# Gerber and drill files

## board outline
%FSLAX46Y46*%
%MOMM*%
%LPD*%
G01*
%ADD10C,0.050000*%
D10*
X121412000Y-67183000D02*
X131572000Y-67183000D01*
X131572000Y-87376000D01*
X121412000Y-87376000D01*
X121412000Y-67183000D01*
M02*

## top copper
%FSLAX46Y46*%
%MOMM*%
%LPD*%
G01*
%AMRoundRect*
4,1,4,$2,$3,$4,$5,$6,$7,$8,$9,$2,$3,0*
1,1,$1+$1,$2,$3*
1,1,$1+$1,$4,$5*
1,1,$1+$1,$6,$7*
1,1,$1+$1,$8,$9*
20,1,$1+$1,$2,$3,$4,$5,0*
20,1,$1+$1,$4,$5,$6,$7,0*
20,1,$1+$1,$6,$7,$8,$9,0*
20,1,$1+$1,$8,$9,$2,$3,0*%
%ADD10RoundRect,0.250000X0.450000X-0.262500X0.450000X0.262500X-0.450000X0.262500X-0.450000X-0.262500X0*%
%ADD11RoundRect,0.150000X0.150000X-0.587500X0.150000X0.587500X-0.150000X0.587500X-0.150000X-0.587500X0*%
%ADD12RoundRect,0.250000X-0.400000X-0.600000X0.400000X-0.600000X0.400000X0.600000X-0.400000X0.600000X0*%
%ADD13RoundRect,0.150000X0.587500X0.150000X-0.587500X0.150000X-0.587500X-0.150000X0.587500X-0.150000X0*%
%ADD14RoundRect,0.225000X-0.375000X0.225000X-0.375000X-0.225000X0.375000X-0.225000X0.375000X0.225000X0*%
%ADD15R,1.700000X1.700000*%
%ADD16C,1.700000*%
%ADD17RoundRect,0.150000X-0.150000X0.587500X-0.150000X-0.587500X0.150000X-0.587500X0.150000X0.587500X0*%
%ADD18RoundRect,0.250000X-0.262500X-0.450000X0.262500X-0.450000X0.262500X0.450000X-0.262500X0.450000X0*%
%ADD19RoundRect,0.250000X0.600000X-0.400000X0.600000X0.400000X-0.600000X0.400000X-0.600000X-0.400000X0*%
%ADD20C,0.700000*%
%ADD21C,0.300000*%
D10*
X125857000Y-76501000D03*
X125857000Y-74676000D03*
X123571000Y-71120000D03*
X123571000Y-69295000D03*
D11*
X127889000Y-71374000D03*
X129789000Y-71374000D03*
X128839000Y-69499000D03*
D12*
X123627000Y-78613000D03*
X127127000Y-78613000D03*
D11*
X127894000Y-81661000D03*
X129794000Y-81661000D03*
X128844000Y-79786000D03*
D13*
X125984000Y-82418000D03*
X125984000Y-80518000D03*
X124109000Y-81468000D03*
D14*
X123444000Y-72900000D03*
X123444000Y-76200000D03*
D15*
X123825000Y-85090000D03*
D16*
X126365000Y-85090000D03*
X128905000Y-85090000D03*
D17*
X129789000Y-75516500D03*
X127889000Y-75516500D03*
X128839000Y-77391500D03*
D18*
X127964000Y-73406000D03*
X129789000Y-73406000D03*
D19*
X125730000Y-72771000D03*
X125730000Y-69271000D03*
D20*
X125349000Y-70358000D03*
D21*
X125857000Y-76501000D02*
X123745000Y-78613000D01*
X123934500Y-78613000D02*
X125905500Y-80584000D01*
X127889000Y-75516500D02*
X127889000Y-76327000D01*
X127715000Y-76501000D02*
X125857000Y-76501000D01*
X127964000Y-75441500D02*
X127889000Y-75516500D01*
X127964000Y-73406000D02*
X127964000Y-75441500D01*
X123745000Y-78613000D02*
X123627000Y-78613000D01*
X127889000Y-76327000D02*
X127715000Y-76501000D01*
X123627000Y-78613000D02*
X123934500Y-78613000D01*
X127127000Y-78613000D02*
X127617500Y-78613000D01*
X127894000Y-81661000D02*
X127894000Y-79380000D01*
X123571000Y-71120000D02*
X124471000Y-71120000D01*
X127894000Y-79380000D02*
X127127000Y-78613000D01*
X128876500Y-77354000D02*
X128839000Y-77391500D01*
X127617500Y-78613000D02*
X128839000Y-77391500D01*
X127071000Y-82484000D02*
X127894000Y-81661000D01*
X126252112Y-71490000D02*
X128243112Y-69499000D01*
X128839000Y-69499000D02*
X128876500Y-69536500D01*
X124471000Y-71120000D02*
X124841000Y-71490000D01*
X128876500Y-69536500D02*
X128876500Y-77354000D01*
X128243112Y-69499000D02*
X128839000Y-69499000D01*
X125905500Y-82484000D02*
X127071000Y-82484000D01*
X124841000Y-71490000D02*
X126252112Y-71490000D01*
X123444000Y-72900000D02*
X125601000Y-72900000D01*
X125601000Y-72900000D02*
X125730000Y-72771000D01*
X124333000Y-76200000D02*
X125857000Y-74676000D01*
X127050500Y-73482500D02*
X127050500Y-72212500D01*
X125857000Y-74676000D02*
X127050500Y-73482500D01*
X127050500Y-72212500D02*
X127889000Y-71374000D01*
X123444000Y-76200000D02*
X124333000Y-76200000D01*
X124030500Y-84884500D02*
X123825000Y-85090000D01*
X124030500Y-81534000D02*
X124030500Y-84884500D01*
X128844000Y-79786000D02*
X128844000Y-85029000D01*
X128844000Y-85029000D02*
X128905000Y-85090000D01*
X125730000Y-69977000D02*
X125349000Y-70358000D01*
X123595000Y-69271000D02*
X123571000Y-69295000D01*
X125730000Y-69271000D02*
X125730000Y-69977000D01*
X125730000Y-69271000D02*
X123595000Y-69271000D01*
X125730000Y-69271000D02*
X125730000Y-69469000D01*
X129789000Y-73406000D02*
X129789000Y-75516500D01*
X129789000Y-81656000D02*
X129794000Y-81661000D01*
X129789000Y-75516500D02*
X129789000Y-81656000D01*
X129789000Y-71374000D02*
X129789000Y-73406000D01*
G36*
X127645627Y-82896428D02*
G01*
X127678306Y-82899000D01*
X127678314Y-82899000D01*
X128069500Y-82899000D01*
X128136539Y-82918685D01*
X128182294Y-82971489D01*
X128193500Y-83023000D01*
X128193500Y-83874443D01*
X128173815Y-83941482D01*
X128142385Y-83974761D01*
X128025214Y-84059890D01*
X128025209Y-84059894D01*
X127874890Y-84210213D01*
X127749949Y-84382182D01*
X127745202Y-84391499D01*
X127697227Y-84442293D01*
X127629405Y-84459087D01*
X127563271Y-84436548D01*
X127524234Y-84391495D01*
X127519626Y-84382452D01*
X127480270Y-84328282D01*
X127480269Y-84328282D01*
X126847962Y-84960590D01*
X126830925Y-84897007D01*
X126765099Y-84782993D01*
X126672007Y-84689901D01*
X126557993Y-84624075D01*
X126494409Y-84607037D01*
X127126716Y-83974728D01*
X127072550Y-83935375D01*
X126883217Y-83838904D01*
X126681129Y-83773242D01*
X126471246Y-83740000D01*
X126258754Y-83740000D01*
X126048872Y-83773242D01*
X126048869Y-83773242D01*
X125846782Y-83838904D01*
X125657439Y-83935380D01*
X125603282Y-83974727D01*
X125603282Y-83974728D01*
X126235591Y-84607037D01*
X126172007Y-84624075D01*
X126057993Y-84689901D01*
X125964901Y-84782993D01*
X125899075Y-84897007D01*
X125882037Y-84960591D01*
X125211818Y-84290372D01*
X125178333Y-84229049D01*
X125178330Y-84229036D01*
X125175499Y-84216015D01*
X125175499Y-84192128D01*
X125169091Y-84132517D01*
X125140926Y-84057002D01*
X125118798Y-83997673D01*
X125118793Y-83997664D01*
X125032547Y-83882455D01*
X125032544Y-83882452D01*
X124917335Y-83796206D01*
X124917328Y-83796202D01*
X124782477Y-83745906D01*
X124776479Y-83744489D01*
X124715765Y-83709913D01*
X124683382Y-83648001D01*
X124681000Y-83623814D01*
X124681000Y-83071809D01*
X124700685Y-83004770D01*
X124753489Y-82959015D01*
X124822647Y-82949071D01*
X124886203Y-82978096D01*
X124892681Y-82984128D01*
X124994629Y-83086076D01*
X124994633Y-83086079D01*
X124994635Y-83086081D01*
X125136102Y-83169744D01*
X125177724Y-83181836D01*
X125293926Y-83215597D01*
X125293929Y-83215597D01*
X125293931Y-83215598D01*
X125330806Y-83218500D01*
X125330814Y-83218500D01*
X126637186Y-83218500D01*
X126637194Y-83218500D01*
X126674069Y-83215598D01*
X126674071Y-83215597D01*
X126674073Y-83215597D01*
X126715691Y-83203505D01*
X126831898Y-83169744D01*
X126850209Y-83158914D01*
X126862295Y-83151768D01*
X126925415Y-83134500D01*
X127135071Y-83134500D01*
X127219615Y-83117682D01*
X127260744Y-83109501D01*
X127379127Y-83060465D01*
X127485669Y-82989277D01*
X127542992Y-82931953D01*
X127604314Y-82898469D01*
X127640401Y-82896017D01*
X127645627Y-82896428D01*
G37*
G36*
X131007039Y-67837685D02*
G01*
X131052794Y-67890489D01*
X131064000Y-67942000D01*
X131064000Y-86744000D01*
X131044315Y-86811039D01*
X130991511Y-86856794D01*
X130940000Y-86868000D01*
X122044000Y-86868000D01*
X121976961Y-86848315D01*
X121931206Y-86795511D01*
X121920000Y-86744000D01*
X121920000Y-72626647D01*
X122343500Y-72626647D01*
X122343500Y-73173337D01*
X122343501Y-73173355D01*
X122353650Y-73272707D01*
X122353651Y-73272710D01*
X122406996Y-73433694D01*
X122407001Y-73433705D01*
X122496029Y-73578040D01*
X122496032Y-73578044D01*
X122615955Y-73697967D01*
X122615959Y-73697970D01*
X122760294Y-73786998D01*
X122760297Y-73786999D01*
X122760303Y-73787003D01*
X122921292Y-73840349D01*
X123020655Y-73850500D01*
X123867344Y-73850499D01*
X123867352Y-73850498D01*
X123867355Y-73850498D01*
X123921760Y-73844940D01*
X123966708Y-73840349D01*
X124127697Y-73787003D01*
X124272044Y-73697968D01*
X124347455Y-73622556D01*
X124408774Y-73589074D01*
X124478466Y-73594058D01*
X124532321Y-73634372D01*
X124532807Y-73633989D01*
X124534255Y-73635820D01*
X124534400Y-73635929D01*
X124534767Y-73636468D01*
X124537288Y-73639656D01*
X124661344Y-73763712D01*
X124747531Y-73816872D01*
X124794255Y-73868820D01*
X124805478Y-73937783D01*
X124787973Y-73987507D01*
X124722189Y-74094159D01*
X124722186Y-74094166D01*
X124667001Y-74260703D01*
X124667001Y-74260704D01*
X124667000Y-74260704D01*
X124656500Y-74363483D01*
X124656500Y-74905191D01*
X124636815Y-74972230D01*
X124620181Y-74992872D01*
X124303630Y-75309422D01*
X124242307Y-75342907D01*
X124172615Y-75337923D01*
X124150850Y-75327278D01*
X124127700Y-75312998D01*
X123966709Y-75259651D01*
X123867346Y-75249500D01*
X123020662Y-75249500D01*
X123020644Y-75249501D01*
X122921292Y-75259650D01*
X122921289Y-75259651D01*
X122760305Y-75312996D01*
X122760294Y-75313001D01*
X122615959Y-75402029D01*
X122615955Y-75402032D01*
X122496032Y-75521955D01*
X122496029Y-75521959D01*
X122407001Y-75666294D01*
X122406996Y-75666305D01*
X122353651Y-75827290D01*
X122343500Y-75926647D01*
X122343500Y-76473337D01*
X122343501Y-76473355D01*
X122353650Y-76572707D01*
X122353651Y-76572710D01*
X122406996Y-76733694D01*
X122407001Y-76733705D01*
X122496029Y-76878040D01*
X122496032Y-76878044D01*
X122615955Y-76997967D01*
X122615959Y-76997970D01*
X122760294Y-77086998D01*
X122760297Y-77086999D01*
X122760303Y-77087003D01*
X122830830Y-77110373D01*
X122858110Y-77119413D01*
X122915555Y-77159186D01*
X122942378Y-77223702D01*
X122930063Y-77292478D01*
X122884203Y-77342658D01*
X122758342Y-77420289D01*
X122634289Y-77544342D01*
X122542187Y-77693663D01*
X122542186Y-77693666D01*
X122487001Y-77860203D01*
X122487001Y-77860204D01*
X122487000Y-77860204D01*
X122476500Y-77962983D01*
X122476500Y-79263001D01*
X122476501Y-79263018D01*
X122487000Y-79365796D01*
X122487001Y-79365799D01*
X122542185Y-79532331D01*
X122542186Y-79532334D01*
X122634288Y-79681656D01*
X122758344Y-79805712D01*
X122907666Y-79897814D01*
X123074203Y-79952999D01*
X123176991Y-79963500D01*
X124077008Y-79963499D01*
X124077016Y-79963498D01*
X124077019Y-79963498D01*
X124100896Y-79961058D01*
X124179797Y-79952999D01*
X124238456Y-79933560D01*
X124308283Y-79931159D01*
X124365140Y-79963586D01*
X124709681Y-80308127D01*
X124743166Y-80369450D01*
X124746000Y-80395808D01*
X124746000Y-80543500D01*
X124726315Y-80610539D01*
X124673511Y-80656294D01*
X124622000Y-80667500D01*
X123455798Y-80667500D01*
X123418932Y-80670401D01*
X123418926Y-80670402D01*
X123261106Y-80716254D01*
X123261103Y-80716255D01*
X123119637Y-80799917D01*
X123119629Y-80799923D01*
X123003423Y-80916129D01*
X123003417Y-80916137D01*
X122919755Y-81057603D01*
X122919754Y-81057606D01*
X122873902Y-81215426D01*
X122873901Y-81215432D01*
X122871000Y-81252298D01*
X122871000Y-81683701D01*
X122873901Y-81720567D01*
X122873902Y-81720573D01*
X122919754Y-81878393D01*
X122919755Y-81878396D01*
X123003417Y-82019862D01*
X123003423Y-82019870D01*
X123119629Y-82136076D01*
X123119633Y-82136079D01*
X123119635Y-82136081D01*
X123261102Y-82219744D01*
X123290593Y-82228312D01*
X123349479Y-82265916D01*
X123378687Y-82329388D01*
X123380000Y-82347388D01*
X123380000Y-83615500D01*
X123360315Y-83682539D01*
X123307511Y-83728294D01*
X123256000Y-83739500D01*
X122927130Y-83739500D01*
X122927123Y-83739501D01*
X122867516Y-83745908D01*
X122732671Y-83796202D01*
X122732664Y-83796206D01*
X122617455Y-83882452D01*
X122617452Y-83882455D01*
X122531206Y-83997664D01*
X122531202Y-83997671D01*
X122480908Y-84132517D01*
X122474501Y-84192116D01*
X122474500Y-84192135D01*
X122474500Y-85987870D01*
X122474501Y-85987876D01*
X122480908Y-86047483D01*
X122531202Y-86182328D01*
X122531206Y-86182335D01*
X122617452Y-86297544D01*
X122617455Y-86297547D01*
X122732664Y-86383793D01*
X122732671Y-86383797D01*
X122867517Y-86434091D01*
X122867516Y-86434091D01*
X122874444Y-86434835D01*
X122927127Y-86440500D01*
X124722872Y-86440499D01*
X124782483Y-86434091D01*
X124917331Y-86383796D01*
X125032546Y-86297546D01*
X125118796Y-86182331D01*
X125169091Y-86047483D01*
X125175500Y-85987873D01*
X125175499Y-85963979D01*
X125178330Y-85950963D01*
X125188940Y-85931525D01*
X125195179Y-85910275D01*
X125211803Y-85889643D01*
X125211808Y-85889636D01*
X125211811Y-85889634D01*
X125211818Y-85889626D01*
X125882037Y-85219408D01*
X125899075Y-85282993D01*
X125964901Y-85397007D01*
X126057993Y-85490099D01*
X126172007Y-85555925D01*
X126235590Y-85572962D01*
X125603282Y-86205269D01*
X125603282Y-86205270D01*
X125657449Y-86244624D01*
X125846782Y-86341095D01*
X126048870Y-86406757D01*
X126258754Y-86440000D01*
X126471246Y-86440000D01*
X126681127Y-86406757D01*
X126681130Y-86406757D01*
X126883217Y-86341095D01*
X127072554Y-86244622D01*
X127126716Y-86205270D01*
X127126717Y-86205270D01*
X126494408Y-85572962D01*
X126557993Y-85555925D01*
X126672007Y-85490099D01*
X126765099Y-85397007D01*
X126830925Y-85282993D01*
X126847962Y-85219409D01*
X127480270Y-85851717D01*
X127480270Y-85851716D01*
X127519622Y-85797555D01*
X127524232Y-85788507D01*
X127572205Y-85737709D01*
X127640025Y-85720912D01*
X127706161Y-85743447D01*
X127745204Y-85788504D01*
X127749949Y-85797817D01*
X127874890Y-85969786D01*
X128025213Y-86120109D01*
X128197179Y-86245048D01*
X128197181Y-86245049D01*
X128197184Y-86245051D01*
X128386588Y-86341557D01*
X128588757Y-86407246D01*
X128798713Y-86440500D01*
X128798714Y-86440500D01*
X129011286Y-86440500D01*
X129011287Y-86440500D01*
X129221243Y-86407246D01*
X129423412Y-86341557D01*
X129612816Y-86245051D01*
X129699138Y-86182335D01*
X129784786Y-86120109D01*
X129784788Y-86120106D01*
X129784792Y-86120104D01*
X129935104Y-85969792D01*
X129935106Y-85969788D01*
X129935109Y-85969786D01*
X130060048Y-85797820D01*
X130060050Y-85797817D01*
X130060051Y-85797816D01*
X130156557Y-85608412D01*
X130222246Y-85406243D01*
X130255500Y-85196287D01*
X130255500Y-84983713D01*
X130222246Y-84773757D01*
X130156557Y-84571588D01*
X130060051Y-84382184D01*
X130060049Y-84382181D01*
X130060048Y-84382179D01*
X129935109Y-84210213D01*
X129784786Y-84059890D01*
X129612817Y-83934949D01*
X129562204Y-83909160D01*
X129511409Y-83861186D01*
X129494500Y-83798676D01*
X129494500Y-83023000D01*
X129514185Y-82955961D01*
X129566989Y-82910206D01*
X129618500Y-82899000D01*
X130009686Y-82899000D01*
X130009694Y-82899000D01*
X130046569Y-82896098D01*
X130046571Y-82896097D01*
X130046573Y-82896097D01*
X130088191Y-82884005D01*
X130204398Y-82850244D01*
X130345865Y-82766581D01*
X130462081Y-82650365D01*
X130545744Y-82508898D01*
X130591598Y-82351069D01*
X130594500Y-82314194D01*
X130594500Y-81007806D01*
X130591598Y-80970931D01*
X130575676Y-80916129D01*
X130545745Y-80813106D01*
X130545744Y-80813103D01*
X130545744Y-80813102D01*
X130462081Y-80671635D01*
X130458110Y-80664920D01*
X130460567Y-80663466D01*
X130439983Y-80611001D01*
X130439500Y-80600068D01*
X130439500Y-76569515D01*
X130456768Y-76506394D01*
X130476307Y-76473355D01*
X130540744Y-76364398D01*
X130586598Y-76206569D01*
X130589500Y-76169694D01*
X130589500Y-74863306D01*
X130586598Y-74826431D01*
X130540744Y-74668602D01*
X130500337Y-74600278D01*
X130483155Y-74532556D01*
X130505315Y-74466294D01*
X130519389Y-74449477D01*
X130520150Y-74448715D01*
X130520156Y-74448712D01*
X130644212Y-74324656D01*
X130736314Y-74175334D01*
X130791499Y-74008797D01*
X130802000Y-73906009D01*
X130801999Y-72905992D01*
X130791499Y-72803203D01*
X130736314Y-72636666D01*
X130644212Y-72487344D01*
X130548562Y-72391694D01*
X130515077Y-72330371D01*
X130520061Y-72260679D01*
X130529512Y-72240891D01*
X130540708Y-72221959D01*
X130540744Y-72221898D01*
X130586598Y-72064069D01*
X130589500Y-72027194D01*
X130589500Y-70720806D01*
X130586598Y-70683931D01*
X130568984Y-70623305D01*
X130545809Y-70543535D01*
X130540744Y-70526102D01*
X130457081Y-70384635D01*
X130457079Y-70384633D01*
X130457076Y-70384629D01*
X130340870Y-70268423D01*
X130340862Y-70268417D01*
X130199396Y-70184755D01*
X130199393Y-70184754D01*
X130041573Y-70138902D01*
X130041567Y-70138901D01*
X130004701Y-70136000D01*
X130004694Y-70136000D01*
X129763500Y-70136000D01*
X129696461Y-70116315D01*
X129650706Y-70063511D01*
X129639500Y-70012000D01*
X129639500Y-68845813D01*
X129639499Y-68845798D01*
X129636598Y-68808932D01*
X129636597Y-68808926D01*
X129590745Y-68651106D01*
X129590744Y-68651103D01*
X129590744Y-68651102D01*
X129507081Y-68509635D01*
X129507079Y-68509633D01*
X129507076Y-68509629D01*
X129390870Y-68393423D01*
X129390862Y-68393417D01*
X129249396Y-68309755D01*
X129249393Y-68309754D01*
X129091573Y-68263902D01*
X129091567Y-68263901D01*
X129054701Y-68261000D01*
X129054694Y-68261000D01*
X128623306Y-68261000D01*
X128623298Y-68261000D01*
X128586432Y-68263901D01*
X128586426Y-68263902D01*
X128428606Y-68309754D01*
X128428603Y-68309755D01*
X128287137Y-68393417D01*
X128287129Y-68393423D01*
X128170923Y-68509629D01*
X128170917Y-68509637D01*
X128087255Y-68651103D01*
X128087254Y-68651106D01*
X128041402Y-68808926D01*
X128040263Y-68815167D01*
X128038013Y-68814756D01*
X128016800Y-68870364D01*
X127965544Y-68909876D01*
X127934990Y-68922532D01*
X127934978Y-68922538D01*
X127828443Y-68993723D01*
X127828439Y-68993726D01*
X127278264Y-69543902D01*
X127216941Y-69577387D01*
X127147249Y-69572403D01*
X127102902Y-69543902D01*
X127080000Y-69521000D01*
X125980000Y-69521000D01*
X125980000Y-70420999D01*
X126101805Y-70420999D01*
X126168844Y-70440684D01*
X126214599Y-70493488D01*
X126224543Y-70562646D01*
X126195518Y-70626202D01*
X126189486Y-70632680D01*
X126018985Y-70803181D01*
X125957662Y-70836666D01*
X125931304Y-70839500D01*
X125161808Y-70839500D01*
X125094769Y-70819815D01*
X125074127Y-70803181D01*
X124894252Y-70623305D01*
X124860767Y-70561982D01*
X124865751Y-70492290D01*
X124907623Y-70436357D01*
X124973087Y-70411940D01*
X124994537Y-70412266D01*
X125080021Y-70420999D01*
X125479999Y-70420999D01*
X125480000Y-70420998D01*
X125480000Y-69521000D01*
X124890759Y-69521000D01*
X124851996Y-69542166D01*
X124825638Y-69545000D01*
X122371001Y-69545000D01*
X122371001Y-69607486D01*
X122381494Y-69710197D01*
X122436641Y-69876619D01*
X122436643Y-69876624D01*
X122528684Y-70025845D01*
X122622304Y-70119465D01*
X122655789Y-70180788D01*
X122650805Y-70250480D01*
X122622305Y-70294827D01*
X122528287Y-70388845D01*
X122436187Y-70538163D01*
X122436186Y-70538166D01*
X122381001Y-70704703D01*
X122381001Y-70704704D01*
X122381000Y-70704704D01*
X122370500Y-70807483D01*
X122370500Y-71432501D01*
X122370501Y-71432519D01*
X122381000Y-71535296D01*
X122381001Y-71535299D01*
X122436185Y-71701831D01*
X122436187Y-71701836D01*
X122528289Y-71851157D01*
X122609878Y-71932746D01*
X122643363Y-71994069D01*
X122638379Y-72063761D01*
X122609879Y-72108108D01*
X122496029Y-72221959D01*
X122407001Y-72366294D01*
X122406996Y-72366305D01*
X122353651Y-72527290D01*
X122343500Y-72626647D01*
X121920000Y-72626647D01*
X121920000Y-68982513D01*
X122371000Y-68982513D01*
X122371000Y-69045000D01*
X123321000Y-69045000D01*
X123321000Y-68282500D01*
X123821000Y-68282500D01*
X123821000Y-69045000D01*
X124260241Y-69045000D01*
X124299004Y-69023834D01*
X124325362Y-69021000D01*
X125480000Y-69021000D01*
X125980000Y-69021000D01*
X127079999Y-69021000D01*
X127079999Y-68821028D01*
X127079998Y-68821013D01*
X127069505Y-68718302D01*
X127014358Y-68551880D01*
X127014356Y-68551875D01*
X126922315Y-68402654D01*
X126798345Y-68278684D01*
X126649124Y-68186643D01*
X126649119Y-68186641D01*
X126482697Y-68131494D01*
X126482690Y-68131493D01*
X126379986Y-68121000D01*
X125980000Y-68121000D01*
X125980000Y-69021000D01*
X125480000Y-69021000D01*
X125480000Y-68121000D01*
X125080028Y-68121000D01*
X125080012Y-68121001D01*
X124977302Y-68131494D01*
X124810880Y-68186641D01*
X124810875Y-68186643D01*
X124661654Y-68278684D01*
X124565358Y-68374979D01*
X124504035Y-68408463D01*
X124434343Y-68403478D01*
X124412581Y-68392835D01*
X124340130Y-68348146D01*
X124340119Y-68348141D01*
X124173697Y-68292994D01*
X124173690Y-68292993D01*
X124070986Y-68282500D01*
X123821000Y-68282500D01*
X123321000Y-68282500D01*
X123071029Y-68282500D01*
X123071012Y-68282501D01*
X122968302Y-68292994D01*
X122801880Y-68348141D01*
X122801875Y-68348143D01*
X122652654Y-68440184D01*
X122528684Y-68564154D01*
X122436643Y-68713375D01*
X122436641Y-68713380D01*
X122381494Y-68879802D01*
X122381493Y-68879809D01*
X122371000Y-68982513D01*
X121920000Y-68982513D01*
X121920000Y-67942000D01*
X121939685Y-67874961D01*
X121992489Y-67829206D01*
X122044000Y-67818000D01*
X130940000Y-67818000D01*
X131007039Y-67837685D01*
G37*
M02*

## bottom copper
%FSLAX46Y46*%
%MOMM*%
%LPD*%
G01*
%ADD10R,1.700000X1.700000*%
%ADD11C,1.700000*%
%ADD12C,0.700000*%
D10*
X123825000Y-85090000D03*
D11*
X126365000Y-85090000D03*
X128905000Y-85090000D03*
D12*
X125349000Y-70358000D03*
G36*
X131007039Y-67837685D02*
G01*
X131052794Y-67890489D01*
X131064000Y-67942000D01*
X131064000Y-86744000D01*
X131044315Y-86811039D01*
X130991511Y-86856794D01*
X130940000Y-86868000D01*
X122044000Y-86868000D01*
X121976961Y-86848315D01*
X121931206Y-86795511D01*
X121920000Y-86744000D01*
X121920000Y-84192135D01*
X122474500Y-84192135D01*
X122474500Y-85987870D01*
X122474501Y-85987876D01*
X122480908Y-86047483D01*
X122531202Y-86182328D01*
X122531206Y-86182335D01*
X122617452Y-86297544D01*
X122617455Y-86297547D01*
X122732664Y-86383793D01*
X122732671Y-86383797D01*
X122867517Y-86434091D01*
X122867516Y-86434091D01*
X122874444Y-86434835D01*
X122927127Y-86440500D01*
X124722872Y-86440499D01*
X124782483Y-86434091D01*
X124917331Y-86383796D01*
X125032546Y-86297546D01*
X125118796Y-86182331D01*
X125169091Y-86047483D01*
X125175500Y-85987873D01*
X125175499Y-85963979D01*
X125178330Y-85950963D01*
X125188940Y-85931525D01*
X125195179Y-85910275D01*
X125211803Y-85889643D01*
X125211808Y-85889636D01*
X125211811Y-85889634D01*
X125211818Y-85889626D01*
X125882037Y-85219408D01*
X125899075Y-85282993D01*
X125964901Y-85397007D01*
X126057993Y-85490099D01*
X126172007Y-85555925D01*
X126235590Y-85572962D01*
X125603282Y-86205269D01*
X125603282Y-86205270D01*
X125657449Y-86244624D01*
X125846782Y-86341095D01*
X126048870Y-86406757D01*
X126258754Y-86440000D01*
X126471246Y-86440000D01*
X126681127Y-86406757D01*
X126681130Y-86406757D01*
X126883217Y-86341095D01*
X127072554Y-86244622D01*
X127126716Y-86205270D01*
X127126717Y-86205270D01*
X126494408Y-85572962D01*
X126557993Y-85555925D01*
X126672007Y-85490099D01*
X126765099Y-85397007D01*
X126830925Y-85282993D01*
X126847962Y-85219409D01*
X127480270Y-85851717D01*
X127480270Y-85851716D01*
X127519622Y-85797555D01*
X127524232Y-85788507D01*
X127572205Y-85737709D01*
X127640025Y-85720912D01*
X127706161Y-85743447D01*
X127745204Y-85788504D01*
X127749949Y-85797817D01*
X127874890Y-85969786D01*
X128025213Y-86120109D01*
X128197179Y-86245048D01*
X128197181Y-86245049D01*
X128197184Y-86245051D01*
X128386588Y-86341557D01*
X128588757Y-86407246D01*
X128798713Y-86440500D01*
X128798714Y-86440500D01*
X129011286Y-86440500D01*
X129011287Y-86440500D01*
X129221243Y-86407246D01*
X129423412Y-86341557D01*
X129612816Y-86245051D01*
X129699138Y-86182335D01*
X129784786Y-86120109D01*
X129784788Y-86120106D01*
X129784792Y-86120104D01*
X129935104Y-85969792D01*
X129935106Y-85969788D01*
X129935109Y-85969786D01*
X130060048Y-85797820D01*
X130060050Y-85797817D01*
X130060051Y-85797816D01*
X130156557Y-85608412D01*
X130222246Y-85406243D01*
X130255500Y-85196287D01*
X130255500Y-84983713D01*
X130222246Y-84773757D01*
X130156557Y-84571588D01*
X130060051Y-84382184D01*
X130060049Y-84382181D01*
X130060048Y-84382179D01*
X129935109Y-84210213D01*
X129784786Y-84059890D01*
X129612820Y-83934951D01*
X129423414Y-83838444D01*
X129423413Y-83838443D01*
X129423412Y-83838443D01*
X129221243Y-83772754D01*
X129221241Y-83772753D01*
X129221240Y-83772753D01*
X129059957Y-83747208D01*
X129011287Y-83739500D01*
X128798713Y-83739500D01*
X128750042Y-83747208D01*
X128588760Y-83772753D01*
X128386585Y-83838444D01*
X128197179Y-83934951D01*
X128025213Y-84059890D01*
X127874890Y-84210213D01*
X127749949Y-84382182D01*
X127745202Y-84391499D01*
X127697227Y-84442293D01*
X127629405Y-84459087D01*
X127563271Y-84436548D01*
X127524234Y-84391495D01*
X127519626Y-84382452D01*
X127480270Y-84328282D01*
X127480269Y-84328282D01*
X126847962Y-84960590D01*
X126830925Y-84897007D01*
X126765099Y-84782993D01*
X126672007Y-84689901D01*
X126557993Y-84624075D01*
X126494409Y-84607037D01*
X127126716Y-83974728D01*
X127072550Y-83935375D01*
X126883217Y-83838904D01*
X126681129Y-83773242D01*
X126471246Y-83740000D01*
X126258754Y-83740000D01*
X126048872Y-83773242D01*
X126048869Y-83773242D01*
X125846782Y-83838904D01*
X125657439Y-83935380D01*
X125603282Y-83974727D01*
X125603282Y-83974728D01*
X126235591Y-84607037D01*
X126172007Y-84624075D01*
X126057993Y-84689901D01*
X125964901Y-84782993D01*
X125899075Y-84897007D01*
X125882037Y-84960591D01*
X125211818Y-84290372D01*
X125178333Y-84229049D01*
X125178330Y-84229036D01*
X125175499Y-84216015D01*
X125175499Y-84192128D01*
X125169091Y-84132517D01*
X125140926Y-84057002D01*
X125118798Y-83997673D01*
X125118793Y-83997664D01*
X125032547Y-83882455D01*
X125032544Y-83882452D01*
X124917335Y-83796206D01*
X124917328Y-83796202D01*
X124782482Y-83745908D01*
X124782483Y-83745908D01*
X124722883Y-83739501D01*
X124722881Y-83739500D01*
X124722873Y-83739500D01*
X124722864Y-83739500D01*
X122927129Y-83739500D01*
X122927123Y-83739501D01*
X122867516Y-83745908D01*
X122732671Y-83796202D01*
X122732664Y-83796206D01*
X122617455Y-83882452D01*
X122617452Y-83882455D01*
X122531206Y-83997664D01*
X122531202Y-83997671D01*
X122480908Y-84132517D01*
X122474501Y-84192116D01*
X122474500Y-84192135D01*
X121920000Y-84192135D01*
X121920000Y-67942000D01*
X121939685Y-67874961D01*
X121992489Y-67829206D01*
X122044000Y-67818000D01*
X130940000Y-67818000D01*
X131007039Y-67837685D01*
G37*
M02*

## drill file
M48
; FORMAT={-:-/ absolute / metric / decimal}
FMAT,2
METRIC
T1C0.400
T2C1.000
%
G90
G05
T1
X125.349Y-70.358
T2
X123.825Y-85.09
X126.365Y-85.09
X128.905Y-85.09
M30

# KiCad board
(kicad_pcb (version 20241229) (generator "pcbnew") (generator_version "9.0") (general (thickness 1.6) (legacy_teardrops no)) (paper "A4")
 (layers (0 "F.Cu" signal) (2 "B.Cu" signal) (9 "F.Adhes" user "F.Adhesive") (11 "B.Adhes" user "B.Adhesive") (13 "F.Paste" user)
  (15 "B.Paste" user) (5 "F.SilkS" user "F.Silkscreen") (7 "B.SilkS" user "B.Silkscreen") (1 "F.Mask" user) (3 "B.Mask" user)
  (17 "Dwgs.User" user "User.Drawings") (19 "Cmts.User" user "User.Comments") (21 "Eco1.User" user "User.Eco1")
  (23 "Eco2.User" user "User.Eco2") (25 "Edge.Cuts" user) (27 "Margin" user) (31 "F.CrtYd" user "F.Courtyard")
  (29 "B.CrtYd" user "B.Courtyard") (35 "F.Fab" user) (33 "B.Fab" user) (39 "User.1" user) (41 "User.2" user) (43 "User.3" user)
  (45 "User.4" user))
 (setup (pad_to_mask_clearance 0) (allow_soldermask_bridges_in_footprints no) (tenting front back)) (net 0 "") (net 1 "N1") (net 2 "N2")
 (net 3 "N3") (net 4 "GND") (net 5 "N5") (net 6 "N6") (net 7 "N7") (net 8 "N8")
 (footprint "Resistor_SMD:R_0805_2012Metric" (layer "F.Cu") (at 125.857 75.5885 90)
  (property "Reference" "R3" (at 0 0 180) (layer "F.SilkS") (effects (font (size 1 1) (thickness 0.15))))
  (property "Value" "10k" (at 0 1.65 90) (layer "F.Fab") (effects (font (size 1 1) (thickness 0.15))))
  (pad "1" smd roundrect (at -0.9125 0 90) (size 1.025 1.4) (layers "F.Cu" "F.Mask" "F.Paste") (roundrect_rratio 0.243902) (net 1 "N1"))
  (pad "2" smd roundrect (at 0.9125 0 90) (size 1.025 1.4) (layers "F.Cu" "F.Mask" "F.Paste") (roundrect_rratio 0.243902) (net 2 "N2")))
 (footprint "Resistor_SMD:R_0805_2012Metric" (layer "F.Cu") (at 123.571 70.2075 90)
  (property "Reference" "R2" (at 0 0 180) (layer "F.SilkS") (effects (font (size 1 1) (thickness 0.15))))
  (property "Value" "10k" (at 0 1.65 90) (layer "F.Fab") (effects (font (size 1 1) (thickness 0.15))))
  (pad "1" smd roundrect (at -0.9125 0 90) (size 1.025 1.4) (layers "F.Cu" "F.Mask" "F.Paste") (roundrect_rratio 0.243902) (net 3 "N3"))
  (pad "2" smd roundrect (at 0.9125 0 90) (size 1.025 1.4) (layers "F.Cu" "F.Mask" "F.Paste") (roundrect_rratio 0.243902) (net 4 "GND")))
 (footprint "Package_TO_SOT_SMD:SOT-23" (layer "F.Cu") (at 128.839 70.4365 90)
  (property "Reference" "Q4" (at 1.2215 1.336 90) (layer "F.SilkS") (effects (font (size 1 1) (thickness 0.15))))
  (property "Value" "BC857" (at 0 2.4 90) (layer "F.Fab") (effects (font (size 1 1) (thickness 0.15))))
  (pad "1" smd roundrect (at -0.9375 -0.95 90) (size 1.475 0.6) (layers "F.Cu" "F.Mask" "F.Paste") (roundrect_rratio 0.25) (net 2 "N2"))
  (pad "2" smd roundrect (at -0.9375 0.95 90) (size 1.475 0.6) (layers "F.Cu" "F.Mask" "F.Paste") (roundrect_rratio 0.25) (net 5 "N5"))
  (pad "3" smd roundrect (at 0.9375 0 90) (size 1.475 0.6) (layers "F.Cu" "F.Mask" "F.Paste") (roundrect_rratio 0.25) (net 3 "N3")))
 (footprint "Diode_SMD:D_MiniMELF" (layer "F.Cu") (at 125.377 78.613)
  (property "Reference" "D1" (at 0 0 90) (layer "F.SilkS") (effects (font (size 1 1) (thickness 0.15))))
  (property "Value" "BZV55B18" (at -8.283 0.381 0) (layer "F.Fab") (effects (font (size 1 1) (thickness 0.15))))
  (pad "1" smd roundrect (at -1.75 0) (size 1.3 1.7) (layers "F.Cu" "F.Mask" "F.Paste") (roundrect_rratio 0.1923076923) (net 1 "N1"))
  (pad "2" smd roundrect (at 1.75 0) (size 1.3 1.7) (layers "F.Cu" "F.Mask" "F.Paste") (roundrect_rratio 0.1923076923) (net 3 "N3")))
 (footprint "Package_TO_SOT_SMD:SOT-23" (layer "F.Cu") (at 128.844 80.7235 90)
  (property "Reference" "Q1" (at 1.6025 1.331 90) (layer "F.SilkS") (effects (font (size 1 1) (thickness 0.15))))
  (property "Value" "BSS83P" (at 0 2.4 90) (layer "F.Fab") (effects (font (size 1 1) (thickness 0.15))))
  (pad "1" smd roundrect (at -0.9375 -0.95 90) (size 1.475 0.6) (layers "F.Cu" "F.Mask" "F.Paste") (roundrect_rratio 0.25) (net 3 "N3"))
  (pad "2" smd roundrect (at -0.9375 0.95 90) (size 1.475 0.6) (layers "F.Cu" "F.Mask" "F.Paste") (roundrect_rratio 0.25) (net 5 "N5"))
  (pad "3" smd roundrect (at 0.9375 0 90) (size 1.475 0.6) (layers "F.Cu" "F.Mask" "F.Paste") (roundrect_rratio 0.25) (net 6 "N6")))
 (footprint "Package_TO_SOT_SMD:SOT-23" (layer "F.Cu") (at 125.0465 81.468 180)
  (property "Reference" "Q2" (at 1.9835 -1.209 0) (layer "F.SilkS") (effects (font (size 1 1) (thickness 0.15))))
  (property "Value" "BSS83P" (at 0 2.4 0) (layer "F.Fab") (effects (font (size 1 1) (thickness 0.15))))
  (pad "1" smd roundrect (at -0.9375 -0.95 180) (size 1.475 0.6) (layers "F.Cu" "F.Mask" "F.Paste") (roundrect_rratio 0.25) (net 3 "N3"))
  (pad "2" smd roundrect (at -0.9375 0.95 180) (size 1.475 0.6) (layers "F.Cu" "F.Mask" "F.Paste") (roundrect_rratio 0.25) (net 1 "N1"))
  (pad "3" smd roundrect (at 0.9375 0 180) (size 1.475 0.6) (layers "F.Cu" "F.Mask" "F.Paste") (roundrect_rratio 0.25) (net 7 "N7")))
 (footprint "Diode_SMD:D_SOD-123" (layer "F.Cu") (at 123.444 74.55 -90)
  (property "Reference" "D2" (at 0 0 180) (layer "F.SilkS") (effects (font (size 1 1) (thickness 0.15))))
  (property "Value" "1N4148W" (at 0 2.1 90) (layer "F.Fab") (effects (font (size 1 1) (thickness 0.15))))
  (pad "1" smd roundrect (at -1.65 0 270) (size 0.9 1.2) (layers "F.Cu" "F.Mask" "F.Paste") (roundrect_rratio 0.25) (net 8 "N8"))
  (pad "2" smd roundrect (at 1.65 0 270) (size 0.9 1.2) (layers "F.Cu" "F.Mask" "F.Paste") (roundrect_rratio 0.25) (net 2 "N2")))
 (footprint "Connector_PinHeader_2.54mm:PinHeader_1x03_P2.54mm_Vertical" (layer "F.Cu") (at 123.825 85.09 90)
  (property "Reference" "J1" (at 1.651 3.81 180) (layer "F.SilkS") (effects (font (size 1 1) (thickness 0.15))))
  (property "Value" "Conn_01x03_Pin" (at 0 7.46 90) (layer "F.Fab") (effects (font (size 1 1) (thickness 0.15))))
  (pad "1" thru_hole rect (at 0 0 90) (size 1.7 1.7) (drill 1) (layers "*.Cu" "*.Mask") (remove_unused_layers no) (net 7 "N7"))
  (pad "2" thru_hole circle (at 0 2.54 90) (size 1.7 1.7) (drill 1) (layers "*.Cu" "*.Mask") (remove_unused_layers no) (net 4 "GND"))
  (pad "3" thru_hole circle (at 0 5.08 90) (size 1.7 1.7) (drill 1) (layers "*.Cu" "*.Mask") (remove_unused_layers no) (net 6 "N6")))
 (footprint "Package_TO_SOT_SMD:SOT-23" (layer "F.Cu") (at 128.839 76.454 -90)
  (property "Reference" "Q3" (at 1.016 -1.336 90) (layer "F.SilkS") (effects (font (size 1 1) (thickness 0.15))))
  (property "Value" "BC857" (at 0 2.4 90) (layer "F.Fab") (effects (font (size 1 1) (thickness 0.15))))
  (pad "1" smd roundrect (at -0.9375 -0.95 270) (size 1.475 0.6) (layers "F.Cu" "F.Mask" "F.Paste") (roundrect_rratio 0.25) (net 5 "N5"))
  (pad "2" smd roundrect (at -0.9375 0.95 270) (size 1.475 0.6) (layers "F.Cu" "F.Mask" "F.Paste") (roundrect_rratio 0.25) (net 1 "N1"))
  (pad "3" smd roundrect (at 0.9375 0 270) (size 1.475 0.6) (layers "F.Cu" "F.Mask" "F.Paste") (roundrect_rratio 0.25) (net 3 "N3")))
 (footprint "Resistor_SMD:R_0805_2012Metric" (layer "F.Cu") (at 128.8765 73.406)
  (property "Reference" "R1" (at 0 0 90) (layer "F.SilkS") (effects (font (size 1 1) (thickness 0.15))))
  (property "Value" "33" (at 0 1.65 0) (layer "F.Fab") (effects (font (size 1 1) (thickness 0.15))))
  (pad "1" smd roundrect (at -0.9125 0) (size 1.025 1.4) (layers "F.Cu" "F.Mask" "F.Paste") (roundrect_rratio 0.243902) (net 1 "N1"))
  (pad "2" smd roundrect (at 0.9125 0) (size 1.025 1.4) (layers "F.Cu" "F.Mask" "F.Paste") (roundrect_rratio 0.243902) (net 5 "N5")))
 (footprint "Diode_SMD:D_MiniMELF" (layer "F.Cu") (at 125.73 71.021 90)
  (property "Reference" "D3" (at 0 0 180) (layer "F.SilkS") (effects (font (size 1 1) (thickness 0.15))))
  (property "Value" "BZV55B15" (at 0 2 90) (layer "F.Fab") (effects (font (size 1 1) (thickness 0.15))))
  (pad "1" smd roundrect (at -1.75 0 90) (size 1.3 1.7) (layers "F.Cu" "F.Mask" "F.Paste") (roundrect_rratio 0.1923076923) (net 8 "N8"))
  (pad "2" smd roundrect (at 1.75 0 90) (size 1.3 1.7) (layers "F.Cu" "F.Mask" "F.Paste") (roundrect_rratio 0.1923076923) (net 4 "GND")))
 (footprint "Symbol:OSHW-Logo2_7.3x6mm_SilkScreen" (layer "B.Cu") (at 126.492 78.359 180)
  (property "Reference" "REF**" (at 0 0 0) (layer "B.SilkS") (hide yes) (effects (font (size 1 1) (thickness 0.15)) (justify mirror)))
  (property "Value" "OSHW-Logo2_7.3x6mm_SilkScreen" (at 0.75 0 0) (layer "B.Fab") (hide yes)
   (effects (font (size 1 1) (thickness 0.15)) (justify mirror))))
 (gr_rect (start 121.412 67.183) (end 131.572 87.376) (stroke (width 0.05) (type default)) (fill no) (layer "Edge.Cuts"))
 (segment (start 125.857 76.501) (end 123.745 78.613) (width 0.3) (layer "F.Cu") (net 1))
 (segment (start 123.9345 78.613) (end 125.9055 80.584) (width 0.3) (layer "F.Cu") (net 1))
 (segment (start 127.889 75.5165) (end 127.889 76.327) (width 0.3) (layer "F.Cu") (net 1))
 (segment (start 127.715 76.501) (end 125.857 76.501) (width 0.3) (layer "F.Cu") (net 1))
 (segment (start 127.964 75.4415) (end 127.889 75.5165) (width 0.3) (layer "F.Cu") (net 1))
 (segment (start 127.964 73.406) (end 127.964 75.4415) (width 0.3) (layer "F.Cu") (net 1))
 (segment (start 123.745 78.613) (end 123.627 78.613) (width 0.3) (layer "F.Cu") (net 1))
 (segment (start 127.889 76.327) (end 127.715 76.501) (width 0.3) (layer "F.Cu") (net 1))
 (segment (start 123.627 78.613) (end 123.9345 78.613) (width 0.3) (layer "F.Cu") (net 1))
 (segment (start 127.127 78.613) (end 127.6175 78.613) (width 0.3) (layer "F.Cu") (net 3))
 (segment (start 127.894 81.661) (end 127.894 79.38) (width 0.3) (layer "F.Cu") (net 3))
 (segment (start 123.571 71.12) (end 124.471 71.12) (width 0.3) (layer "F.Cu") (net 3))
 (segment (start 127.894 79.38) (end 127.127 78.613) (width 0.3) (layer "F.Cu") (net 3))
 (segment (start 128.8765 77.354) (end 128.839 77.3915) (width 0.3) (layer "F.Cu") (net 3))
 (segment (start 127.6175 78.613) (end 128.839 77.3915) (width 0.3) (layer "F.Cu") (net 3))
 (segment (start 127.071 82.484) (end 127.894 81.661) (width 0.3) (layer "F.Cu") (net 3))
 (segment (start 126.252112 71.49) (end 128.243112 69.499) (width 0.3) (layer "F.Cu") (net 3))
 (segment (start 128.839 69.499) (end 128.8765 69.5365) (width 0.3) (layer "F.Cu") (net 3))
 (segment (start 124.471 71.12) (end 124.841 71.49) (width 0.3) (layer "F.Cu") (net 3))
 (segment (start 128.8765 69.5365) (end 128.8765 77.354) (width 0.3) (layer "F.Cu") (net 3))
 (segment (start 128.243112 69.499) (end 128.839 69.499) (width 0.3) (layer "F.Cu") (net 3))
 (segment (start 125.9055 82.484) (end 127.071 82.484) (width 0.3) (layer "F.Cu") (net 3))
 (segment (start 124.841 71.49) (end 126.252112 71.49) (width 0.3) (layer "F.Cu") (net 3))
 (segment (start 123.444 72.9) (end 125.601 72.9) (width 0.3) (layer "F.Cu") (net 8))
 (segment (start 125.601 72.9) (end 125.73 72.771) (width 0.3) (layer "F.Cu") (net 8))
 (segment (start 124.333 76.2) (end 125.857 74.676) (width 0.3) (layer "F.Cu") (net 2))
 (segment (start 127.0505 73.4825) (end 127.0505 72.2125) (width 0.3) (layer "F.Cu") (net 2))
 (segment (start 125.857 74.676) (end 127.0505 73.4825) (width 0.3) (layer "F.Cu") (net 2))
 (segment (start 127.0505 72.2125) (end 127.889 71.374) (width 0.3) (layer "F.Cu") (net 2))
 (segment (start 123.444 76.2) (end 124.333 76.2) (width 0.3) (layer "F.Cu") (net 2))
 (segment (start 124.0305 84.8845) (end 123.825 85.09) (width 0.3) (layer "F.Cu") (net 7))
 (segment (start 124.0305 81.534) (end 124.0305 84.8845) (width 0.3) (layer "F.Cu") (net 7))
 (segment (start 128.844 79.786) (end 128.844 85.029) (width 0.3) (layer "F.Cu") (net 6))
 (segment (start 128.844 85.029) (end 128.905 85.09) (width 0.3) (layer "F.Cu") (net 6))
 (segment (start 125.73 69.977) (end 125.349 70.358) (width 0.3) (layer "F.Cu") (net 4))
 (segment (start 123.595 69.271) (end 123.571 69.295) (width 0.3) (layer "F.Cu") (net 4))
 (segment (start 125.73 69.271) (end 125.73 69.977) (width 0.3) (layer "F.Cu") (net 4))
 (segment (start 125.73 69.271) (end 123.595 69.271) (width 0.3) (layer "F.Cu") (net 4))
 (segment (start 125.73 69.271) (end 125.73 69.469) (width 0.3) (layer "F.Cu") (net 4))
 (via (at 125.349 70.358) (size 0.7) (drill 0.4) (layers "F.Cu" "B.Cu") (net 4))
 (segment (start 129.789 73.406) (end 129.789 75.5165) (width 0.3) (layer "F.Cu") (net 5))
 (segment (start 129.789 81.656) (end 129.794 81.661) (width 0.3) (layer "F.Cu") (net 5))
 (segment (start 129.789 75.5165) (end 129.789 81.656) (width 0.3) (layer "F.Cu") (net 5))
 (segment (start 129.789 71.374) (end 129.789 73.406) (width 0.3) (layer "F.Cu") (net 5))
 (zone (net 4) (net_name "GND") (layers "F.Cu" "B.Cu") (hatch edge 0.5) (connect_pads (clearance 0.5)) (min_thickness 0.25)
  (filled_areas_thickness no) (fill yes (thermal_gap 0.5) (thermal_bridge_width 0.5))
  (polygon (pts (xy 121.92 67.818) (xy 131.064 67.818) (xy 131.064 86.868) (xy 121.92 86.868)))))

